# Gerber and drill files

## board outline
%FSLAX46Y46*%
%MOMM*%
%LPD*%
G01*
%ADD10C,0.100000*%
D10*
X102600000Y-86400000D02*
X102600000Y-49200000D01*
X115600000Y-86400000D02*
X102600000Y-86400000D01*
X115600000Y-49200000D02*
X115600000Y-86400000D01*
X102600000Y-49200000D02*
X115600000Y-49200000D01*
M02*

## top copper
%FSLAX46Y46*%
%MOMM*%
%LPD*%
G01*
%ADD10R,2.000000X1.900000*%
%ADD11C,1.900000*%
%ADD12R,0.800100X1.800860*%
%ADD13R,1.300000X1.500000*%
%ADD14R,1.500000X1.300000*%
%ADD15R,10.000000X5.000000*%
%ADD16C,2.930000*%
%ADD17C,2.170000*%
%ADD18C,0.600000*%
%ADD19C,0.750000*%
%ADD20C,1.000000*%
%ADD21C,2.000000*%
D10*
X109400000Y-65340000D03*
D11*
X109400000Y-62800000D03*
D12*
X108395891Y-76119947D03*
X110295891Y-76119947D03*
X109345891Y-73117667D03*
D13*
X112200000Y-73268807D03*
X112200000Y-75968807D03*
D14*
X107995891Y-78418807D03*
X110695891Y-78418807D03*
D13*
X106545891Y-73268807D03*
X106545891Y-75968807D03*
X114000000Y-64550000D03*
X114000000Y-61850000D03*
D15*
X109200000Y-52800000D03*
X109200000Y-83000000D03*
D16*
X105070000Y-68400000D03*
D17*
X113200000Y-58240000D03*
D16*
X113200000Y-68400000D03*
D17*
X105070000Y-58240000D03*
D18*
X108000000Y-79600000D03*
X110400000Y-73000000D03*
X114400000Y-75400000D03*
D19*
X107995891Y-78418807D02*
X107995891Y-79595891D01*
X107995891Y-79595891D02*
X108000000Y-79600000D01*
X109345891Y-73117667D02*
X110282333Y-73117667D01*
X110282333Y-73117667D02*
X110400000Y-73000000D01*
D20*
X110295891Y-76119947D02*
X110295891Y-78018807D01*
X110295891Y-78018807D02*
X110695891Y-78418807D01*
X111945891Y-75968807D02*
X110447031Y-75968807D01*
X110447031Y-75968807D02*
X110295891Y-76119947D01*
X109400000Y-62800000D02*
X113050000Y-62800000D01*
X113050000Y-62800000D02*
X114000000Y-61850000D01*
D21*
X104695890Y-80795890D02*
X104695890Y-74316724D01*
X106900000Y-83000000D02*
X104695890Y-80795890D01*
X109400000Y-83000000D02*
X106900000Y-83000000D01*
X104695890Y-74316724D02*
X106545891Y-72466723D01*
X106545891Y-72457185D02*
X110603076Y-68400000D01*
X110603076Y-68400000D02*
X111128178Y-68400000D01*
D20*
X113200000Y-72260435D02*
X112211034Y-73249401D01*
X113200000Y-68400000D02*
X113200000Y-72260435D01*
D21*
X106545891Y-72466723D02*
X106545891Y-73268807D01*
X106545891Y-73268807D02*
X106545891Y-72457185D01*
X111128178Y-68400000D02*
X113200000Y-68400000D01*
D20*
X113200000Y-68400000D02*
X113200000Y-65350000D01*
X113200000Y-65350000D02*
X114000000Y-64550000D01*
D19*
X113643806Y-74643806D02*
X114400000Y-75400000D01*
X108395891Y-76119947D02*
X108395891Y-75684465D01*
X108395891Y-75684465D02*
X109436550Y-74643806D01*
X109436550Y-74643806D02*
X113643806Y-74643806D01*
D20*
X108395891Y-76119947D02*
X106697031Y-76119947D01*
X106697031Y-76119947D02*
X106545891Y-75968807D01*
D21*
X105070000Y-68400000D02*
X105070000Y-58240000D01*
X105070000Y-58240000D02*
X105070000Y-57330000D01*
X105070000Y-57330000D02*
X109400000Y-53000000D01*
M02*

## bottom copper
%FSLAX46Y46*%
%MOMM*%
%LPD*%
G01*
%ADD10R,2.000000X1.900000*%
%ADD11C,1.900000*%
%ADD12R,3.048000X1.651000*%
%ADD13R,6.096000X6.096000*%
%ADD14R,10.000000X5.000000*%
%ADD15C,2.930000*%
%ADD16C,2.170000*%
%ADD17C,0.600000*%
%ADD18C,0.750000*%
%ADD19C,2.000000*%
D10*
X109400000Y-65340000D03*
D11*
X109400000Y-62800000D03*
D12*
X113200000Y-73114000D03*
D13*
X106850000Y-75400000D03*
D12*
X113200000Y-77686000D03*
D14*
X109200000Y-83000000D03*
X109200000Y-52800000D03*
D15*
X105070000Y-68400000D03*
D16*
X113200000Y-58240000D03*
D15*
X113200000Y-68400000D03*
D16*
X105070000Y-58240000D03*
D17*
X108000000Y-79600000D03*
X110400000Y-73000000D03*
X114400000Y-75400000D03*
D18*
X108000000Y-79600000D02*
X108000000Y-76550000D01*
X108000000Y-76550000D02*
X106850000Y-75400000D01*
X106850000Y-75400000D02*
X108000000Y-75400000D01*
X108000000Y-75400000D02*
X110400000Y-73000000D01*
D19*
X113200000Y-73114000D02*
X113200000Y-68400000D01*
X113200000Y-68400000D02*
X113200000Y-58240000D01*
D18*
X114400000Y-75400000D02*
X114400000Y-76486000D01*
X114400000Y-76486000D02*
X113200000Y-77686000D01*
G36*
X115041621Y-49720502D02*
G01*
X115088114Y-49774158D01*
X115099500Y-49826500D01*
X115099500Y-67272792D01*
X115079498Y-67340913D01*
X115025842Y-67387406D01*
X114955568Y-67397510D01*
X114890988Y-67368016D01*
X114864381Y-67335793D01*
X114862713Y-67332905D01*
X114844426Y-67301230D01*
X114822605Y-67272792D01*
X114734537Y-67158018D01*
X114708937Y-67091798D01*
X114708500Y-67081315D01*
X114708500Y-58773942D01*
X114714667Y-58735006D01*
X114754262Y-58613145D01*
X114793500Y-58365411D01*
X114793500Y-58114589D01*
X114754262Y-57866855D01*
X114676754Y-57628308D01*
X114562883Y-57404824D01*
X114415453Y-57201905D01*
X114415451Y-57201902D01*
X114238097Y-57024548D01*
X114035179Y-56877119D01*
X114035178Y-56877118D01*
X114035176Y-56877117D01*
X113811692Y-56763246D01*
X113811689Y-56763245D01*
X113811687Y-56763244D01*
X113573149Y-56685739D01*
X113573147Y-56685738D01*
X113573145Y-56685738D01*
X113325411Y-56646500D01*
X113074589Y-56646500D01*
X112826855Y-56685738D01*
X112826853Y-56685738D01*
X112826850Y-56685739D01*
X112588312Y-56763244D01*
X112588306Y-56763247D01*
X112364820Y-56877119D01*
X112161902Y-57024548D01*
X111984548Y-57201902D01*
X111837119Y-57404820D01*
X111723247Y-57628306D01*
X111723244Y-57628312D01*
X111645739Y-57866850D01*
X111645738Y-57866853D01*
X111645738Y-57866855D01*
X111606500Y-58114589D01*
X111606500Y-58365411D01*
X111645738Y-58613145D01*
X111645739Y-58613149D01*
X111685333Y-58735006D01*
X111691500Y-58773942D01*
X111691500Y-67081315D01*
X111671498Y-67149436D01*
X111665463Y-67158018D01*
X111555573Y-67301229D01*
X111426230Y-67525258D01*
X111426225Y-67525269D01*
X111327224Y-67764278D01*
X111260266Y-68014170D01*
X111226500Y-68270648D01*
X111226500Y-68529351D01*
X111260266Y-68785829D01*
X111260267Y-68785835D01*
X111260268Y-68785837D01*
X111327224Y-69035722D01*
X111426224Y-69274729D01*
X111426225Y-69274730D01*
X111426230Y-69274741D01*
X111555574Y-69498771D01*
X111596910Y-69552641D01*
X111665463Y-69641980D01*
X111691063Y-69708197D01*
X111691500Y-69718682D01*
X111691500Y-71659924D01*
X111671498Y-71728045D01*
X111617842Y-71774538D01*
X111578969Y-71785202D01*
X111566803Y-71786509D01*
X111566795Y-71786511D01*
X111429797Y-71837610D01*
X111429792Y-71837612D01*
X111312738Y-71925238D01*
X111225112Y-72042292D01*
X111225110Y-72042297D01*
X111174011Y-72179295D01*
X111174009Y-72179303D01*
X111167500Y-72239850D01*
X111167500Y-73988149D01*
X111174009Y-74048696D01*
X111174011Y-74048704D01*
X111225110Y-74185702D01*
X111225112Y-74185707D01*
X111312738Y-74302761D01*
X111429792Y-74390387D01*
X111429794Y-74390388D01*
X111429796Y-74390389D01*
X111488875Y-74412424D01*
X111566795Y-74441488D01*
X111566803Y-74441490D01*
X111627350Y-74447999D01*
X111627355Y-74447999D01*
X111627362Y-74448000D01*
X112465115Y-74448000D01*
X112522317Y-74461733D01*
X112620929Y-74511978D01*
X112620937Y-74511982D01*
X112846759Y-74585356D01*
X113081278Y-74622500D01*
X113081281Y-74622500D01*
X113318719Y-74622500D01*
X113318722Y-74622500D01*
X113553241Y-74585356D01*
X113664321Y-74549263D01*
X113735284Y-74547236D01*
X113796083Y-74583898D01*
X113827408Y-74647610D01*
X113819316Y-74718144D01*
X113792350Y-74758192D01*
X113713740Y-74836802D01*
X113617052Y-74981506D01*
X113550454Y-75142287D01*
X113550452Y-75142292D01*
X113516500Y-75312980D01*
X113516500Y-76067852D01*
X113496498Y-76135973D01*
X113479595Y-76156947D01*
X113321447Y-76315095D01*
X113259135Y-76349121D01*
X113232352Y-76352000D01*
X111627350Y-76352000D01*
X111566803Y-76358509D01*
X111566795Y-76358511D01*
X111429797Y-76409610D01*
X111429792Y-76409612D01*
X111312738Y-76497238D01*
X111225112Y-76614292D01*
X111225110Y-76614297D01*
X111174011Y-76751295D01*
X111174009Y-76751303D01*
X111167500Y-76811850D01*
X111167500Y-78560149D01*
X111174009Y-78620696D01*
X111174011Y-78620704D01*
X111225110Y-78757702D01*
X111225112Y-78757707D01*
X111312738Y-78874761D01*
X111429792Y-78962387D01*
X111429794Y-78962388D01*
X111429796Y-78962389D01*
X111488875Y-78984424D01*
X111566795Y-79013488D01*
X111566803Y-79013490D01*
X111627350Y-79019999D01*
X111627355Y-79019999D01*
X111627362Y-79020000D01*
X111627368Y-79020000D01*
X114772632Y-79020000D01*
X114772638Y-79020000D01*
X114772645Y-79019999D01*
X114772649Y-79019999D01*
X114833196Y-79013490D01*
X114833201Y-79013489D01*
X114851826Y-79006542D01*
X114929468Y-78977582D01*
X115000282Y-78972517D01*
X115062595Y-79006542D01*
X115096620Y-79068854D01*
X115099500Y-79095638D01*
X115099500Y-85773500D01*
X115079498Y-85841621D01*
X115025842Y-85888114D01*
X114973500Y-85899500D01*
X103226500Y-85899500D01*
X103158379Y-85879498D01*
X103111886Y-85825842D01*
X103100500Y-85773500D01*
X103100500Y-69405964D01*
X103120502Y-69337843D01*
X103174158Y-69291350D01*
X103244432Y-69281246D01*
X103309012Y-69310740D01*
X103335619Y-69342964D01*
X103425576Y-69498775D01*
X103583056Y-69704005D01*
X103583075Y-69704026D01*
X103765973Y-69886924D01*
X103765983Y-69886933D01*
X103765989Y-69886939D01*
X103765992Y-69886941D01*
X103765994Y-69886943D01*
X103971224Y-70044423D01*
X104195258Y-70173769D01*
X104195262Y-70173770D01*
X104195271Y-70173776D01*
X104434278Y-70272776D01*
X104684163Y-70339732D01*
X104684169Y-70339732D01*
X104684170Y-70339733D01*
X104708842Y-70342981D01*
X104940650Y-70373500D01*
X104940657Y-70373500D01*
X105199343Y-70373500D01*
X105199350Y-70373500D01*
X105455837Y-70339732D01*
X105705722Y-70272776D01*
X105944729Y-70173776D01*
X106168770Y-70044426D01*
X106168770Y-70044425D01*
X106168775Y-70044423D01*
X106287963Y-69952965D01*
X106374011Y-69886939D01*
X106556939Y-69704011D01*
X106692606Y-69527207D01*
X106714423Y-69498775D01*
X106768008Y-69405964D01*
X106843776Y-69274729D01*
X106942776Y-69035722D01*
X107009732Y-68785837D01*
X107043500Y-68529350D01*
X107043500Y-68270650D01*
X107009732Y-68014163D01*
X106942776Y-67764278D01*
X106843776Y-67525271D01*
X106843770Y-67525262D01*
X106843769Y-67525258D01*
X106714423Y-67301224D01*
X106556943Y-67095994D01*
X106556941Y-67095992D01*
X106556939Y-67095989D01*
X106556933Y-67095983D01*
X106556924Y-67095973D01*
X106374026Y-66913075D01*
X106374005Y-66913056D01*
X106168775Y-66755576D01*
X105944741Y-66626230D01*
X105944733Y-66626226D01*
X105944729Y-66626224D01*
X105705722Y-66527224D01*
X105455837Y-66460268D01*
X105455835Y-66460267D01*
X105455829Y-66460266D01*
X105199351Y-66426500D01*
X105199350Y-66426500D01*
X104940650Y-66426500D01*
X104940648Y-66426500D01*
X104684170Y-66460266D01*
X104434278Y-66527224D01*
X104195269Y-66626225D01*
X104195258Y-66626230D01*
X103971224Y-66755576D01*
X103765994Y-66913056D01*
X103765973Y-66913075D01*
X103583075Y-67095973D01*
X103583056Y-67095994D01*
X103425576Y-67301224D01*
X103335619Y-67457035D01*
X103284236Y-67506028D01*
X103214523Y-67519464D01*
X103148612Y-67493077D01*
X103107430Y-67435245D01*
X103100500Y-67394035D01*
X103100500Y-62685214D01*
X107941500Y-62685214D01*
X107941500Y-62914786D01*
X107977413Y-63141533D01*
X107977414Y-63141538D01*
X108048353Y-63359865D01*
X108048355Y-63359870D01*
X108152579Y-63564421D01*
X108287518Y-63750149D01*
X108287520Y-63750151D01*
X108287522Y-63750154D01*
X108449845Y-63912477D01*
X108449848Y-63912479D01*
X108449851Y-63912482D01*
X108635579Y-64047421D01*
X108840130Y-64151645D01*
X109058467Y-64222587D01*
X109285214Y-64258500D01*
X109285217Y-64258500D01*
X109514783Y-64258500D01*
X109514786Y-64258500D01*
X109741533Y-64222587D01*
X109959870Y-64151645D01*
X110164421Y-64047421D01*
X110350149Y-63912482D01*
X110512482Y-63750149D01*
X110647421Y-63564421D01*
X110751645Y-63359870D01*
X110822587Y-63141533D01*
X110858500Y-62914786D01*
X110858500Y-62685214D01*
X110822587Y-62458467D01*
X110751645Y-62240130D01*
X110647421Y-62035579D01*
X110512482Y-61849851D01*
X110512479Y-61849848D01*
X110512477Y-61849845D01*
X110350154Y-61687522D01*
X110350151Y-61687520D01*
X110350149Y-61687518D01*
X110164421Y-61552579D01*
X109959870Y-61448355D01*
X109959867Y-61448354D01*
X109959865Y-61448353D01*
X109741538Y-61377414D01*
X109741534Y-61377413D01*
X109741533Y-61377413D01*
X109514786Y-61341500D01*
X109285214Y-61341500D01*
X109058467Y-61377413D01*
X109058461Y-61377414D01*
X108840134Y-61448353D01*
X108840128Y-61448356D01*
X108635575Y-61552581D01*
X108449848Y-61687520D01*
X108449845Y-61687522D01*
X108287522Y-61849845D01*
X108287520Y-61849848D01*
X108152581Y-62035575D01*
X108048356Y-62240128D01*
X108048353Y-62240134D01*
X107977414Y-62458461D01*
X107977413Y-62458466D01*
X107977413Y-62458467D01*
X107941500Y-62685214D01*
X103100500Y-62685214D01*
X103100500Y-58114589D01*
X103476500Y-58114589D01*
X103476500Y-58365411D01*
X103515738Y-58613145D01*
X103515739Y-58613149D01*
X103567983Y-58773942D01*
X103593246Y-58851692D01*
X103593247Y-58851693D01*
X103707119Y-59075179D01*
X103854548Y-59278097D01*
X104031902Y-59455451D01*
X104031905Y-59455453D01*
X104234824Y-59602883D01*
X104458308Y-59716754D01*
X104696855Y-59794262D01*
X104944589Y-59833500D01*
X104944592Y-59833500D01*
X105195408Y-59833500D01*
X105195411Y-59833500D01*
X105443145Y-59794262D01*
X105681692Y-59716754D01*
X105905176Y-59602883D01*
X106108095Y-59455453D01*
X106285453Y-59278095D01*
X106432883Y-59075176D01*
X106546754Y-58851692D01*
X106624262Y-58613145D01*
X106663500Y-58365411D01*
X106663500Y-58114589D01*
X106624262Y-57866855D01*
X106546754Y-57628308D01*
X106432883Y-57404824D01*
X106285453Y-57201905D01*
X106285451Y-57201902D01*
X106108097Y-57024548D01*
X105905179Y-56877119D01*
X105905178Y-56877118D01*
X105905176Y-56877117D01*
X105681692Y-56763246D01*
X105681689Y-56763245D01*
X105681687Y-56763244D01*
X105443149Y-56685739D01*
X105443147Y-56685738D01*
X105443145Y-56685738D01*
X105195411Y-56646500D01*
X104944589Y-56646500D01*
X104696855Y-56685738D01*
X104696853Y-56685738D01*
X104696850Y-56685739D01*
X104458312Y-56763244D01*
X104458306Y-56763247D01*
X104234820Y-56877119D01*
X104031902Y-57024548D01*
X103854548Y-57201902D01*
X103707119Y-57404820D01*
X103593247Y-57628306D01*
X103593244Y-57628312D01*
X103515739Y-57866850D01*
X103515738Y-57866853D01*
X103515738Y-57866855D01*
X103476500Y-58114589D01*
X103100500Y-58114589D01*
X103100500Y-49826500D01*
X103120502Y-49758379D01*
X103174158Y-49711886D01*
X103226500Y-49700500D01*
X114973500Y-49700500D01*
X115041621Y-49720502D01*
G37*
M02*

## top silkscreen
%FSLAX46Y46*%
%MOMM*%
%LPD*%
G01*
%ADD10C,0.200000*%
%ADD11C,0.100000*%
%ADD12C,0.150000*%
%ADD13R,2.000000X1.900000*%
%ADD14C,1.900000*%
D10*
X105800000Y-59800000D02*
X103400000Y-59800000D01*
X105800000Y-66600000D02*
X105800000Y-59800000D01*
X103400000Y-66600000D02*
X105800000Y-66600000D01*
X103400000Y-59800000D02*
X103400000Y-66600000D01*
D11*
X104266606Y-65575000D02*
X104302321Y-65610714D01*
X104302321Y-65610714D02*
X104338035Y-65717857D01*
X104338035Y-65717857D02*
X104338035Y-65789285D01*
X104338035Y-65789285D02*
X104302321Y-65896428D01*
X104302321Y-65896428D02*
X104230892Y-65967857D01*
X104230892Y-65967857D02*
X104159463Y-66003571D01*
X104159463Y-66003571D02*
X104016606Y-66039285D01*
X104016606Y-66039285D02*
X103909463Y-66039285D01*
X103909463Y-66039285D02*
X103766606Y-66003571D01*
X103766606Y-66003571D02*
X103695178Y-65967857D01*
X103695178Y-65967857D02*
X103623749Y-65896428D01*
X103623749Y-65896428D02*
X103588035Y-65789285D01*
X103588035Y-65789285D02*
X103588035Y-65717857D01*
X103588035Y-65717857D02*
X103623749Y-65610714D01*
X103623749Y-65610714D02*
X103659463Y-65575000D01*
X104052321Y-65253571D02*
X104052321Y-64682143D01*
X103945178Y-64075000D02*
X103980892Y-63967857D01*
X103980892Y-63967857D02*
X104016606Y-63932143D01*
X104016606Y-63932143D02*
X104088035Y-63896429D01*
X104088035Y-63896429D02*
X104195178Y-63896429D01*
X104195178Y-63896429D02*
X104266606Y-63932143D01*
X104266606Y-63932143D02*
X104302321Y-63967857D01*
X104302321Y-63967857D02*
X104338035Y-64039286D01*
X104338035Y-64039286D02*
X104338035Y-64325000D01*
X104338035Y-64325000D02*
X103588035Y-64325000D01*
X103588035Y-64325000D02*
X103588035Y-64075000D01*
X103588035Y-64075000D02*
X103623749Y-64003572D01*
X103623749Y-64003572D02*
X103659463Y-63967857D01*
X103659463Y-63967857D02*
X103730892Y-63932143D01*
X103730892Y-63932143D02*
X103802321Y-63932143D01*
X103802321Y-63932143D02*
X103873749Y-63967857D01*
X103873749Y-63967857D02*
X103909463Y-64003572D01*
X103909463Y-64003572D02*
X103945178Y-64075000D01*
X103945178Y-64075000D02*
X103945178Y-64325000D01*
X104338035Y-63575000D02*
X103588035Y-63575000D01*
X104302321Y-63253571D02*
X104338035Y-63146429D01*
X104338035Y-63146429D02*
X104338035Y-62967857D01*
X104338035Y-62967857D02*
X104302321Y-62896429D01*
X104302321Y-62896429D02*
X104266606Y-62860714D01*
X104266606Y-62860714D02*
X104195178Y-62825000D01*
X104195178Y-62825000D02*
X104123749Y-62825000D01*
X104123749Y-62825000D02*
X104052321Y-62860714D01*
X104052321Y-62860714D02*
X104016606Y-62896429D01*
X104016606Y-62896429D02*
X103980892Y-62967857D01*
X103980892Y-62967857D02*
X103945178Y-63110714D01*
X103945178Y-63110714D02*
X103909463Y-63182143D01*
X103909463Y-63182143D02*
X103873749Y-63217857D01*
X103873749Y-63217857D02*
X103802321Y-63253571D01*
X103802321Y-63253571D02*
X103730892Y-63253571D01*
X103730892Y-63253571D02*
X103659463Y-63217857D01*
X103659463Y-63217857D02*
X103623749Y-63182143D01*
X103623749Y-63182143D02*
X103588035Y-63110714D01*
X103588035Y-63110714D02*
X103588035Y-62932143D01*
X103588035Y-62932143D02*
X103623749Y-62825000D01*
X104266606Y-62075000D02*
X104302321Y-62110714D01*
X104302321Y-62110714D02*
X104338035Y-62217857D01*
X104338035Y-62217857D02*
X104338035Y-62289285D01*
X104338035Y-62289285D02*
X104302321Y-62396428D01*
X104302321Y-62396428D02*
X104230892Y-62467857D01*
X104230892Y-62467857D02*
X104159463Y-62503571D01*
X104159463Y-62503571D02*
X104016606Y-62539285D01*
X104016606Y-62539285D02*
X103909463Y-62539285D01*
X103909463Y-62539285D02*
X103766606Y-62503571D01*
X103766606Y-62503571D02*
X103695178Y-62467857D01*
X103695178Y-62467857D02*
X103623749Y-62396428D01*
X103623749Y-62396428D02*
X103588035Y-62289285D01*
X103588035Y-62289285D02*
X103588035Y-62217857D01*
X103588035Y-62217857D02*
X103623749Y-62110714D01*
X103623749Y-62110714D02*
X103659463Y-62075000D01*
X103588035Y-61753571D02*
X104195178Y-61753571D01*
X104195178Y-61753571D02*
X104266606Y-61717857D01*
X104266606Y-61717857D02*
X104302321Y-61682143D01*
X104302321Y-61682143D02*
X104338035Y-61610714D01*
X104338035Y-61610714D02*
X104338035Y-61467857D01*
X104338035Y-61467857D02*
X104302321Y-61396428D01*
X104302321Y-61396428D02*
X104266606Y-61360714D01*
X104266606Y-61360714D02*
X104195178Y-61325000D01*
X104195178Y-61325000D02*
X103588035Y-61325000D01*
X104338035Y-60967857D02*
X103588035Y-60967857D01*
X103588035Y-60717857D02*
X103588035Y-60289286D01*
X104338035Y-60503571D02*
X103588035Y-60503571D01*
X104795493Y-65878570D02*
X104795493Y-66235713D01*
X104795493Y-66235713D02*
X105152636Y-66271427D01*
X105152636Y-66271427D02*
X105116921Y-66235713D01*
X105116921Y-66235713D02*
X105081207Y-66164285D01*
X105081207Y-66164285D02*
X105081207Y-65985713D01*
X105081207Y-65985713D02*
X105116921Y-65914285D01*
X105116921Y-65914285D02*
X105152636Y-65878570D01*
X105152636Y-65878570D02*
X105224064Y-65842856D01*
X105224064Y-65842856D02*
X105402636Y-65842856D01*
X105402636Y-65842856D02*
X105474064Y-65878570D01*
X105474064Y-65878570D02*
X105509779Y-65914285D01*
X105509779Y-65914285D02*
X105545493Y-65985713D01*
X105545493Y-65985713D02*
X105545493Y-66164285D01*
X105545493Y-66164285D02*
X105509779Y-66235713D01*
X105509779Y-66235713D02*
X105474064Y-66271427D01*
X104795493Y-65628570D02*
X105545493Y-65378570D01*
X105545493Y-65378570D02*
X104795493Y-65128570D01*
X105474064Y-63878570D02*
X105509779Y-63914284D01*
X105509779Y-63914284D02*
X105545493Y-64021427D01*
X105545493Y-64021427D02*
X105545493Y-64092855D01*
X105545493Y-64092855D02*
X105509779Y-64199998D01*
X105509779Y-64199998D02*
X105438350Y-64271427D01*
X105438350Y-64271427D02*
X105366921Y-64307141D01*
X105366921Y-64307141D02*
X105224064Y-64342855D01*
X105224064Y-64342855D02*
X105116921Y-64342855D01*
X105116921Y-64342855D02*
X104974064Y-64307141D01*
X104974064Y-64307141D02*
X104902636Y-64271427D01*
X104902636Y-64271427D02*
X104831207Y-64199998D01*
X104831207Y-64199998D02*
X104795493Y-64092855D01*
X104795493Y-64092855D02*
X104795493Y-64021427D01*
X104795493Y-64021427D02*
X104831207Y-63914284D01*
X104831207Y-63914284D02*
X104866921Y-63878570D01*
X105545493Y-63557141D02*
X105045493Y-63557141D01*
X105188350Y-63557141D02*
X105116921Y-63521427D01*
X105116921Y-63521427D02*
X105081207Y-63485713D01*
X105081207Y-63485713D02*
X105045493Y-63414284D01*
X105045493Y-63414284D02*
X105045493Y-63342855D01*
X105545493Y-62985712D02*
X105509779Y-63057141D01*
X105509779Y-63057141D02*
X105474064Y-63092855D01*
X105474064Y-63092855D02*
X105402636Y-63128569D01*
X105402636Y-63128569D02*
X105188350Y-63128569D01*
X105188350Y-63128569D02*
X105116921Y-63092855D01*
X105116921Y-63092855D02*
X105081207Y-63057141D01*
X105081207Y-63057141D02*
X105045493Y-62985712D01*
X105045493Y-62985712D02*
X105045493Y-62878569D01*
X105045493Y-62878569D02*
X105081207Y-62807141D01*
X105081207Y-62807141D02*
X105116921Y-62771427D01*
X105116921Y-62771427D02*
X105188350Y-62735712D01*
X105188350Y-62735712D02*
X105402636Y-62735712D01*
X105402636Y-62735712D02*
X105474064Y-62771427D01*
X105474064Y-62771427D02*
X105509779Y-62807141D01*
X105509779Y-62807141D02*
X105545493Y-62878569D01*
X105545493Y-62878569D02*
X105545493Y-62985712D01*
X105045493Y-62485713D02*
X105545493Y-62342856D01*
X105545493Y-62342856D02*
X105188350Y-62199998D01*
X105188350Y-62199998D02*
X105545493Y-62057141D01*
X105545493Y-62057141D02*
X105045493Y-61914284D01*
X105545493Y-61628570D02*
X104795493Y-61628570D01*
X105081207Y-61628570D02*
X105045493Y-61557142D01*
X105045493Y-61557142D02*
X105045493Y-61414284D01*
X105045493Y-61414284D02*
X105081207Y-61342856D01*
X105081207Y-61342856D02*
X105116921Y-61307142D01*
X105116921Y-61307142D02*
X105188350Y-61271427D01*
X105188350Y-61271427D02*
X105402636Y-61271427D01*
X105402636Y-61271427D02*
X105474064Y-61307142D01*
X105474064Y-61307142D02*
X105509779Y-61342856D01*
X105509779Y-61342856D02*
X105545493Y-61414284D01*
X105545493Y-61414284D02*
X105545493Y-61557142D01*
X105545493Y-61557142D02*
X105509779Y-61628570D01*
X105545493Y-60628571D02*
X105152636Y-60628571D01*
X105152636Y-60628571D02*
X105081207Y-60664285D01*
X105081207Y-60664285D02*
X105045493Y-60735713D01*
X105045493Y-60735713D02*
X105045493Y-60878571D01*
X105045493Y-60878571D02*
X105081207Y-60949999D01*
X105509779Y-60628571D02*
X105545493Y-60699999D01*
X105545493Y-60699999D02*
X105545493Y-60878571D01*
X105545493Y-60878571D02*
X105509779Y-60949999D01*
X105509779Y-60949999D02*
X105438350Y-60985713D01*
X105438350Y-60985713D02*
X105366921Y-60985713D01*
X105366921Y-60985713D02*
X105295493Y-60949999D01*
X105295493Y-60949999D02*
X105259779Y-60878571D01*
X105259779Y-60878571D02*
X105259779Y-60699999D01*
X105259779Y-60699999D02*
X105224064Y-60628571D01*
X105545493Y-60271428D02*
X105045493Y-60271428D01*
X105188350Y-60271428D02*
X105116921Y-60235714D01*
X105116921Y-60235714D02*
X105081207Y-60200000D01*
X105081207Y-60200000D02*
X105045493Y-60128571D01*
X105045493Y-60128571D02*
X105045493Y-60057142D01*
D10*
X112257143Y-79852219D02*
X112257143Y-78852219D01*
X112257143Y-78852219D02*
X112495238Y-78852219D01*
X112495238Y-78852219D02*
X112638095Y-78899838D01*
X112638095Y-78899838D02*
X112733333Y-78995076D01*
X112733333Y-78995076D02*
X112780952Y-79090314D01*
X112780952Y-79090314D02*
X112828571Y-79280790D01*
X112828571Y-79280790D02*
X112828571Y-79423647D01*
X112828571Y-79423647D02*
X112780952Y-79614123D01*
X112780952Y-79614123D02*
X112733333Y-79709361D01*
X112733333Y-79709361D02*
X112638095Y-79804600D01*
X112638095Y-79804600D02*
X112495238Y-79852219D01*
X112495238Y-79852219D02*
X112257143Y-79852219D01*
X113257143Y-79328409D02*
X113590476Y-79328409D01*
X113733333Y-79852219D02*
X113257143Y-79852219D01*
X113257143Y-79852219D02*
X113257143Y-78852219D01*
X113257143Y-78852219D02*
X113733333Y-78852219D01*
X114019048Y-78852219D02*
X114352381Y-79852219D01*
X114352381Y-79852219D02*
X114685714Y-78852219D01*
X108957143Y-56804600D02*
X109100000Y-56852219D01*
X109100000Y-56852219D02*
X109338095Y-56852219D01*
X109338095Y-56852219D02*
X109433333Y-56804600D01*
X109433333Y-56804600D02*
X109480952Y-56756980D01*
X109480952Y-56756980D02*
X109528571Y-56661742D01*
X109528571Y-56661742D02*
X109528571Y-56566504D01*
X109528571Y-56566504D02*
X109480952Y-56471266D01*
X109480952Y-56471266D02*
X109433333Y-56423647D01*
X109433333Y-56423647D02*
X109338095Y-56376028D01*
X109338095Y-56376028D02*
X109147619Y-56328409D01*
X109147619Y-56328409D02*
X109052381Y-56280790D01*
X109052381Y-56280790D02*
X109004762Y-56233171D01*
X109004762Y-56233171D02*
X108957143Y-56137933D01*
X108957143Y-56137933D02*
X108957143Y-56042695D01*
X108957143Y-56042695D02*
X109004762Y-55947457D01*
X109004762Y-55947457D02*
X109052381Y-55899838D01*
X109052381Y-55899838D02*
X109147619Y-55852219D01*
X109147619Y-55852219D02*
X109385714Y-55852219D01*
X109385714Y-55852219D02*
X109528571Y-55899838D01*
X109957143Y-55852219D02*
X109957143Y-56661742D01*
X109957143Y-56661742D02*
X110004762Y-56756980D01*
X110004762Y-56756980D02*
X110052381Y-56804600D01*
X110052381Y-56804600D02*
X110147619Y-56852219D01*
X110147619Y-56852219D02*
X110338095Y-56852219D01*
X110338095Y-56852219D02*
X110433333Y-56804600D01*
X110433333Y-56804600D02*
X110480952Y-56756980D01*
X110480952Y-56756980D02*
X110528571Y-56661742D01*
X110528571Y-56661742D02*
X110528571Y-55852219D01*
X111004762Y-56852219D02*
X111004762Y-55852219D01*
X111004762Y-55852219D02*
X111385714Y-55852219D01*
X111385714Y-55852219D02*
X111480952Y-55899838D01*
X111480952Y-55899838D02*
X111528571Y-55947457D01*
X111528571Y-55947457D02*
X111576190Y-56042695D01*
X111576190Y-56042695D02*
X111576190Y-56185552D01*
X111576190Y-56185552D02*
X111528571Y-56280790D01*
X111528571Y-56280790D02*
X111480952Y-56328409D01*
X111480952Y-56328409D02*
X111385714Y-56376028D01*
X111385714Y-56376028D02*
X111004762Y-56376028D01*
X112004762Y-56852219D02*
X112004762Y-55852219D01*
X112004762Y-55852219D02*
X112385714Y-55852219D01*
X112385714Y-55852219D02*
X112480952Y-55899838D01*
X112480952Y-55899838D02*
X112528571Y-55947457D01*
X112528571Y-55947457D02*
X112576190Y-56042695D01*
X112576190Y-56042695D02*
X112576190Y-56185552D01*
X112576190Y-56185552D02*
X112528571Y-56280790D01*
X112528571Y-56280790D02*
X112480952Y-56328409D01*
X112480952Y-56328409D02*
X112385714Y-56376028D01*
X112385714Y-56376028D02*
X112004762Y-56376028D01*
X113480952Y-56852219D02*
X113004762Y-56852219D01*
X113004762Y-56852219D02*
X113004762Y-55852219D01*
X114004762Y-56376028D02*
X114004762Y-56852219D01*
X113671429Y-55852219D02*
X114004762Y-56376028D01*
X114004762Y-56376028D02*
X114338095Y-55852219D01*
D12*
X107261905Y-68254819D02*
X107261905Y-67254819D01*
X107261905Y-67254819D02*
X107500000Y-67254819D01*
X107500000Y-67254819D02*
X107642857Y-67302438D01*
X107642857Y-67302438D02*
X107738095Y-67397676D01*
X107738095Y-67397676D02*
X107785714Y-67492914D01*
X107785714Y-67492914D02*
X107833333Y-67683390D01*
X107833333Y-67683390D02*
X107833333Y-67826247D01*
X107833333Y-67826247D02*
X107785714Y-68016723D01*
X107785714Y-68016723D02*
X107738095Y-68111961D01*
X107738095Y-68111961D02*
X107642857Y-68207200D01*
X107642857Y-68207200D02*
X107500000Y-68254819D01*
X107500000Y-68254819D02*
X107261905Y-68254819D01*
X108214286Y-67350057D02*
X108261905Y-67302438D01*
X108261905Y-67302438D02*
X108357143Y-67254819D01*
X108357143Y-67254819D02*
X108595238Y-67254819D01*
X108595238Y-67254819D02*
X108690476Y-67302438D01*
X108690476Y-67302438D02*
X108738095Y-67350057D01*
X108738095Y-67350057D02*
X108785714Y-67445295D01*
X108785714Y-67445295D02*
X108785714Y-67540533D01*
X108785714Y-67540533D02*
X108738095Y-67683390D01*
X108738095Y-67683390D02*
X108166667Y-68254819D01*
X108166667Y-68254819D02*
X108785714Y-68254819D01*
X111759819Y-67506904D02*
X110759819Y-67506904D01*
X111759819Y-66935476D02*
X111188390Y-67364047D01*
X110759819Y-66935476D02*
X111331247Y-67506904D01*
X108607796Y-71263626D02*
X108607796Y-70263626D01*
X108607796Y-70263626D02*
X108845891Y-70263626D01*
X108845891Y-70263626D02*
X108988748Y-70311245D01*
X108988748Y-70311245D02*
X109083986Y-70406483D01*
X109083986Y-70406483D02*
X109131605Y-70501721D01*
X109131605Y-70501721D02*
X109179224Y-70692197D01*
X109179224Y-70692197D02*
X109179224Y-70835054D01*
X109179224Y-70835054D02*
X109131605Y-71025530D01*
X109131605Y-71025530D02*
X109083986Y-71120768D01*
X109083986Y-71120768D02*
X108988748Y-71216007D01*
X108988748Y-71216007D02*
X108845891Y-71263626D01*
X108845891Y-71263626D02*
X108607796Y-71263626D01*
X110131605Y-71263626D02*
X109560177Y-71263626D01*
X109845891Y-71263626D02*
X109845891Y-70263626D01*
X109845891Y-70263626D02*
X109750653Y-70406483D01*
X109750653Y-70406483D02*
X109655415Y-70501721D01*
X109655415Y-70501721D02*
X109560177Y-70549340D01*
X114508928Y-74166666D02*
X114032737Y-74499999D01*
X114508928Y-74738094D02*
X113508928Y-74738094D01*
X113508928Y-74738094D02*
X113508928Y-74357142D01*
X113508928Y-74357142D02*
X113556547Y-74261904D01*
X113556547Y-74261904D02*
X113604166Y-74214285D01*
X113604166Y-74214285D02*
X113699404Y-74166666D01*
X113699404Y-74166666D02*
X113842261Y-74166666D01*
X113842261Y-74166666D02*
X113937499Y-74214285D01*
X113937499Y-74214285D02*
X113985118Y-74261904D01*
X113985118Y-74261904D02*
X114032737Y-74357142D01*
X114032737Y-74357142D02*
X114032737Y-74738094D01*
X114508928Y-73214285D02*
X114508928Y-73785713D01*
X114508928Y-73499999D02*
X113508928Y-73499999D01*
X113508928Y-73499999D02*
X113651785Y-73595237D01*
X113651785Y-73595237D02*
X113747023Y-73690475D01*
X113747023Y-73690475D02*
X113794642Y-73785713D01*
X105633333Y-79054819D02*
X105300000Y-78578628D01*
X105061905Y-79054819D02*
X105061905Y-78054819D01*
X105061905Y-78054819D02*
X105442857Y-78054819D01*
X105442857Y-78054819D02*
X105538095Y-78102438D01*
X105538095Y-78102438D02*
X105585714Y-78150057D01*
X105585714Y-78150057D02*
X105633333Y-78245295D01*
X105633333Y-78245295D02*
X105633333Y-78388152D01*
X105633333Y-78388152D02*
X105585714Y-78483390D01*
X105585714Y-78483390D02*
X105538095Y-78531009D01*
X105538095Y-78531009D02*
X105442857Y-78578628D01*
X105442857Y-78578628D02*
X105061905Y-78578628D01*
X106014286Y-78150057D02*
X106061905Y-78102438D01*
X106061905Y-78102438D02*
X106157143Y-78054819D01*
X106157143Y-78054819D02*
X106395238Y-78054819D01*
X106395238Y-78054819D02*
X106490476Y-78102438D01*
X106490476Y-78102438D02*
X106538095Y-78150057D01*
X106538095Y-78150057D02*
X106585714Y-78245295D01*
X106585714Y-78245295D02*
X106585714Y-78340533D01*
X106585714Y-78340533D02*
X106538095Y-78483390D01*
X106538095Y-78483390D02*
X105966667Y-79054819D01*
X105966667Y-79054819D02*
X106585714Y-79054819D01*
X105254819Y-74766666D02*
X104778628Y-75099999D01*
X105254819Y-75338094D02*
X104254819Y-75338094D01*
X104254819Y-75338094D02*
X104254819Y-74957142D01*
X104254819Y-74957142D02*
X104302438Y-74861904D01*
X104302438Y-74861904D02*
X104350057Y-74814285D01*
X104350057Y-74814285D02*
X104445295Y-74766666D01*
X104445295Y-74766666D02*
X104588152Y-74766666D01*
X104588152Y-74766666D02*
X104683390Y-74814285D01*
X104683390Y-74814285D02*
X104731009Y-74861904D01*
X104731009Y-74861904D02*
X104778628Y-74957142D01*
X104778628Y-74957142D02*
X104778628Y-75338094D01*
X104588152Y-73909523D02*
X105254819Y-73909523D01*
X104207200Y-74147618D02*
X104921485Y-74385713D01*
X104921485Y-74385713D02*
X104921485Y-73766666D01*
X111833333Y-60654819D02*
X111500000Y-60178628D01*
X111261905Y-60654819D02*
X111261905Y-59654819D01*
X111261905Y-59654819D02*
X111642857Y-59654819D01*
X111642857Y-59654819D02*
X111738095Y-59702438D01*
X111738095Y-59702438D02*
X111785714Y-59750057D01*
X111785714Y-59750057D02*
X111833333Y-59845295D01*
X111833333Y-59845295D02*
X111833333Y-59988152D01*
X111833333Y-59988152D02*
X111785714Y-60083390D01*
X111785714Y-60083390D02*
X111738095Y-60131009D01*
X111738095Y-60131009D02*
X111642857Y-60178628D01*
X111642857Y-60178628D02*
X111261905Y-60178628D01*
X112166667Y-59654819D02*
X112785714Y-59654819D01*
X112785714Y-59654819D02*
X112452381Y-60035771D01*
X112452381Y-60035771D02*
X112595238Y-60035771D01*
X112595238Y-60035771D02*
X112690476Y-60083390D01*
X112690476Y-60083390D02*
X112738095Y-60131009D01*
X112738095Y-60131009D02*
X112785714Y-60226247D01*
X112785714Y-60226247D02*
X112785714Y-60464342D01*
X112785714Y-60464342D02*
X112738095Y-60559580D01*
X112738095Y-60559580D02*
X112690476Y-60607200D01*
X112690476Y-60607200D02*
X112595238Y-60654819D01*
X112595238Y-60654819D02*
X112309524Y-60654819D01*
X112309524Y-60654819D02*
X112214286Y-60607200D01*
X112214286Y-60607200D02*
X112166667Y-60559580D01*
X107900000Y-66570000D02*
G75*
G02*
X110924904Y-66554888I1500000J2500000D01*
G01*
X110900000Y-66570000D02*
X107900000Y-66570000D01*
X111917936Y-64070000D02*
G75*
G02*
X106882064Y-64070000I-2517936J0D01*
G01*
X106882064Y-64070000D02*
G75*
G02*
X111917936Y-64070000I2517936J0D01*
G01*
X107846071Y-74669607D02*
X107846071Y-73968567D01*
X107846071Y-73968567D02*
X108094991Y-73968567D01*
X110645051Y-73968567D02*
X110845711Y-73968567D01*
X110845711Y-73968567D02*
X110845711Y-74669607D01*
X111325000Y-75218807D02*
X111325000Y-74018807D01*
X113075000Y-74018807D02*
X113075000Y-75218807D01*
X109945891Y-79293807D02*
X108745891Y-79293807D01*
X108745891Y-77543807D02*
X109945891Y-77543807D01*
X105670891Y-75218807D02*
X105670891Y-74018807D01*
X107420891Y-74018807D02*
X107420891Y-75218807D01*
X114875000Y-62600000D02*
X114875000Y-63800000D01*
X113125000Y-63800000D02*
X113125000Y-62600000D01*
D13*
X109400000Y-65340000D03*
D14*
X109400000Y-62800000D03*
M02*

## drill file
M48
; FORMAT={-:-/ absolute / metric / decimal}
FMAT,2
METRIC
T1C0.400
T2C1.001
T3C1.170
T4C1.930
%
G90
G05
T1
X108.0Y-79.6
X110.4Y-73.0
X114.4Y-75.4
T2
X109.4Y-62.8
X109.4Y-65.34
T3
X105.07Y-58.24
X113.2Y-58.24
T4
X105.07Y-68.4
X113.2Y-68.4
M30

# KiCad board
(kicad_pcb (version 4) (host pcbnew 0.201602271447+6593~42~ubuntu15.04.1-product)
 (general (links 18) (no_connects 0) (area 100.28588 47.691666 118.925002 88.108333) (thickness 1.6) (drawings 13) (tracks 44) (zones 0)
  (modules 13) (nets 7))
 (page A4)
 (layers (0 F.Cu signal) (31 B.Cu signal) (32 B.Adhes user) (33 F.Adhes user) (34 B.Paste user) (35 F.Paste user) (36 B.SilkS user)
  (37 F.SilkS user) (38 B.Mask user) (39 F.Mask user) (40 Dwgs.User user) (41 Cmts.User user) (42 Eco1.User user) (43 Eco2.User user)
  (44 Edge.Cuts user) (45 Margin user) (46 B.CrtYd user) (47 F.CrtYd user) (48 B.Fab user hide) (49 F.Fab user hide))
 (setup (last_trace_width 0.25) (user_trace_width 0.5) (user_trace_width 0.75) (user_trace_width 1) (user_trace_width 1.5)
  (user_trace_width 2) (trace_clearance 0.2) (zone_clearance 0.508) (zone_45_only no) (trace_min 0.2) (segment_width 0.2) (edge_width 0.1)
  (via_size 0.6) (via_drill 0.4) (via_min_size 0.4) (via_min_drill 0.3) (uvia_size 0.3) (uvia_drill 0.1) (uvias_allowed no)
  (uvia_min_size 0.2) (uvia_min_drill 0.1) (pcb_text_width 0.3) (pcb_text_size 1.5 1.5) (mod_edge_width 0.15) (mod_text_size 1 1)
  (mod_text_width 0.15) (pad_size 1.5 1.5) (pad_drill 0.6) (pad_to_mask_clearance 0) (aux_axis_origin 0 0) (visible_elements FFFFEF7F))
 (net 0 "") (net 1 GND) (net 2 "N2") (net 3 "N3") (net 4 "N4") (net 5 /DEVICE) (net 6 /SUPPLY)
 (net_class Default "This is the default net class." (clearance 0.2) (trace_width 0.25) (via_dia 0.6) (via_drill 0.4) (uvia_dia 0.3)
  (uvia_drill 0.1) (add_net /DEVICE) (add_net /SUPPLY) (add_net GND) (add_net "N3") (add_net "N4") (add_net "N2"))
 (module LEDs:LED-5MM (layer F.Cu) (at 109.4 65.34 90)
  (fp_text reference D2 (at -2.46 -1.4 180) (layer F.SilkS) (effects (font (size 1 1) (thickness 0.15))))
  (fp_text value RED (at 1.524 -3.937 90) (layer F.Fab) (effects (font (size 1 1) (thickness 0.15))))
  (fp_arc (start 1.27 0) (end -1.23 -1.5) (angle 297.5) (layer F.SilkS) (width 0.15))
  (fp_line (start -1.23 1.5) (end -1.23 -1.5) (layer F.SilkS) (width 0.15))
  (fp_circle (center 1.27 0) (end 0.97 -2.5) (layer F.SilkS) (width 0.15))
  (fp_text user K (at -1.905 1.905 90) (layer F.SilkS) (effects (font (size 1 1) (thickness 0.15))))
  (pad 1 thru_hole rect (at 0 0 180) (size 2 1.9) (drill 1.00076) (layers *.Cu *.Mask F.SilkS) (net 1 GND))
  (pad 2 thru_hole circle (at 2.54 0 90) (size 1.9 1.9) (drill 1.00076) (layers *.Cu *.Mask F.SilkS) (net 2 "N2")))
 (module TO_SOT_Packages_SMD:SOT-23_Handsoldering (layer F.Cu) (at 109.345891 74.618807)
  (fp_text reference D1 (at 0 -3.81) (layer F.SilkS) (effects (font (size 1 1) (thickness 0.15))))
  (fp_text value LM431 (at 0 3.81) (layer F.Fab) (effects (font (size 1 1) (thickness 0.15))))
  (fp_line (start -1.49982 0.0508) (end -1.49982 -0.65024) (layer F.SilkS) (width 0.15))
  (fp_line (start -1.49982 -0.65024) (end -1.2509 -0.65024) (layer F.SilkS) (width 0.15))
  (fp_line (start 1.29916 -0.65024) (end 1.49982 -0.65024) (layer F.SilkS) (width 0.15))
  (fp_line (start 1.49982 -0.65024) (end 1.49982 0.0508) (layer F.SilkS) (width 0.15))
  (pad 1 smd rect (at -0.95 1.50114) (size 0.8001 1.80086) (layers F.Cu F.Paste F.Mask) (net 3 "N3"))
  (pad 2 smd rect (at 0.95 1.50114) (size 0.8001 1.80086) (layers F.Cu F.Paste F.Mask) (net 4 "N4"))
  (pad 3 smd rect (at 0 -1.50114) (size 0.8001 1.80086) (layers F.Cu F.Paste F.Mask) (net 1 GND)))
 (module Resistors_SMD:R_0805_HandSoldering (layer F.Cu) (at 112.2 74.618807 270)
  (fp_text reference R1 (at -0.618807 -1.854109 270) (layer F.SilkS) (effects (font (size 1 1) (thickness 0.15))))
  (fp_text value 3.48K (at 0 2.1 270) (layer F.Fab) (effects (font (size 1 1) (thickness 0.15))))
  (fp_line (start 0.6 0.875) (end -0.6 0.875) (layer F.SilkS) (width 0.15))
  (fp_line (start -0.6 -0.875) (end 0.6 -0.875) (layer F.SilkS) (width 0.15))
  (pad 1 smd rect (at -1.35 0 270) (size 1.5 1.3) (layers F.Cu F.Paste F.Mask) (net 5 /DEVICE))
  (pad 2 smd rect (at 1.35 0 270) (size 1.5 1.3) (layers F.Cu F.Paste F.Mask) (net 4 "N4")))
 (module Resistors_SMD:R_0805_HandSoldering (layer F.Cu) (at 109.345891 78.418807)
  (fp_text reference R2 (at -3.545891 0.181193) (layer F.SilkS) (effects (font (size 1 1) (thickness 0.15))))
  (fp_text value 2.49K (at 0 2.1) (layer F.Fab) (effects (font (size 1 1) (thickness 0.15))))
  (fp_line (start 0.6 0.875) (end -0.6 0.875) (layer F.SilkS) (width 0.15))
  (fp_line (start -0.6 -0.875) (end 0.6 -0.875) (layer F.SilkS) (width 0.15))
  (pad 1 smd rect (at -1.35 0) (size 1.5 1.3) (layers F.Cu F.Paste F.Mask) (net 1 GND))
  (pad 2 smd rect (at 1.35 0) (size 1.5 1.3) (layers F.Cu F.Paste F.Mask) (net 4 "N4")))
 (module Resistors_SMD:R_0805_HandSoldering (layer F.Cu) (at 106.545891 74.618807 270)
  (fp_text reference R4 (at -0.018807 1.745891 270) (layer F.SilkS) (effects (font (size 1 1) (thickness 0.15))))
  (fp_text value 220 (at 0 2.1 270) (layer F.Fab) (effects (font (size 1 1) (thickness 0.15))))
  (fp_line (start 0.6 0.875) (end -0.6 0.875) (layer F.SilkS) (width 0.15))
  (fp_line (start -0.6 -0.875) (end 0.6 -0.875) (layer F.SilkS) (width 0.15))
  (pad 1 smd rect (at -1.35 0 270) (size 1.5 1.3) (layers F.Cu F.Paste F.Mask) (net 5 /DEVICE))
  (pad 2 smd rect (at 1.35 0 270) (size 1.5 1.3) (layers F.Cu F.Paste F.Mask) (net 3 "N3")))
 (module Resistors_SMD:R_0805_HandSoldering (layer F.Cu) (at 114 63.2 90)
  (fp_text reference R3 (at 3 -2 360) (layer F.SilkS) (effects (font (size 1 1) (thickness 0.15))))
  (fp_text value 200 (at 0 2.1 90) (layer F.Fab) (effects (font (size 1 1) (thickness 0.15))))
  (fp_line (start 0.6 0.875) (end -0.6 0.875) (layer F.SilkS) (width 0.15))
  (fp_line (start -0.6 -0.875) (end 0.6 -0.875) (layer F.SilkS) (width 0.15))
  (pad 1 smd rect (at -1.35 0 90) (size 1.5 1.3) (layers F.Cu F.Paste F.Mask) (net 5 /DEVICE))
  (pad 2 smd rect (at 1.35 0 90) (size 1.5 1.3) (layers F.Cu F.Paste F.Mask) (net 2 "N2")))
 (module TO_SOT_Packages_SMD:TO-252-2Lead (layer B.Cu) (at 113.2 75.4 270)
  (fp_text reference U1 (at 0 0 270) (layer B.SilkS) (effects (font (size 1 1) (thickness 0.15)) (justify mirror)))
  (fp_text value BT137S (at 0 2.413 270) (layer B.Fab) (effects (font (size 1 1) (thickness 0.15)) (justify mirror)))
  (pad 1 smd rect (at -2.286 0 270) (size 1.651 3.048) (layers B.Cu B.Paste B.Mask) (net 5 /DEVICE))
  (pad 2 smd rect (at 0 6.35 270) (size 6.096 6.096) (layers B.Cu B.Paste B.Mask) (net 1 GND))
  (pad 3 smd rect (at 2.286 0 270) (size 1.651 3.048) (layers B.Cu B.Paste B.Mask) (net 3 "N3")))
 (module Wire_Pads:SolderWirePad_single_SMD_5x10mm (layer F.Cu) (at 109.2 52.8 90)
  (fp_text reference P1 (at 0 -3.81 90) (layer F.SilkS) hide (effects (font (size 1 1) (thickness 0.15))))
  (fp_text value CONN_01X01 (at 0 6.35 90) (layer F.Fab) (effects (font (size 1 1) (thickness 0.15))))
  (pad 1 smd rect (at 0 0 90) (size 5 10) (layers F.Cu F.Paste F.Mask) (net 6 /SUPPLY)))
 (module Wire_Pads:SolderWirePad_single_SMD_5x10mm (layer F.Cu) (at 109.2 83 90)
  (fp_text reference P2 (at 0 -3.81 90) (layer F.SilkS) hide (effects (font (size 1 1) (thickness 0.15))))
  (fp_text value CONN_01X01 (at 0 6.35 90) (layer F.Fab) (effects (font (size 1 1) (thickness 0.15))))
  (pad 1 smd rect (at 0 0 90) (size 5 10) (layers F.Cu F.Paste F.Mask) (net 5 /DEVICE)))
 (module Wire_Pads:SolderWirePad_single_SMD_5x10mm (layer B.Cu) (at 109.2 83 90)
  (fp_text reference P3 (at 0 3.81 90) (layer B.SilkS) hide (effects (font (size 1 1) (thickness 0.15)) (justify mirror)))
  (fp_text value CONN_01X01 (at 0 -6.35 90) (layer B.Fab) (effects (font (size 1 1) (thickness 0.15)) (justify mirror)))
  (pad 1 smd rect (at 0 0 90) (size 5 10) (layers B.Cu B.Paste B.Mask) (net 1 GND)))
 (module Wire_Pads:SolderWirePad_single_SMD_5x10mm (layer B.Cu) (at 109.2 52.8 90)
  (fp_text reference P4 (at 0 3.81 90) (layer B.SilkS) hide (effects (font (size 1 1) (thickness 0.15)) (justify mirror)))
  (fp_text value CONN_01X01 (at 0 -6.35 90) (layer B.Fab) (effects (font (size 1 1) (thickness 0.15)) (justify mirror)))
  (pad 1 smd rect (at 0 0 90) (size 5 10) (layers B.Cu B.Paste B.Mask) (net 1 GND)))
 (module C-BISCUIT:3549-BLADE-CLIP (layer B.Cu) (at 109.135 63.32)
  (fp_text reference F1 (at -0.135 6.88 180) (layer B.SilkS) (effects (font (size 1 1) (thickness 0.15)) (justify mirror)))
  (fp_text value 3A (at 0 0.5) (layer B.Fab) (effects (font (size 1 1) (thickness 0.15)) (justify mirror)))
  (pad 1 thru_hole circle (at -4.065 5.08) (size 2.93 2.93) (drill 1.93) (layers *.Cu *.Mask B.SilkS) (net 6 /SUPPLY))
  (pad 2 thru_hole circle (at 4.065 -5.08) (size 2.17 2.17) (drill 1.17) (layers *.Cu *.Mask B.SilkS) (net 5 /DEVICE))
  (pad 2 thru_hole circle (at 4.065 5.08) (size 2.93 2.93) (drill 1.93) (layers *.Cu *.Mask B.SilkS) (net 5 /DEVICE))
  (pad 1 thru_hole circle (at -4.065 -5.08) (size 2.17 2.17) (drill 1.17) (layers *.Cu *.Mask B.SilkS) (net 6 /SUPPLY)))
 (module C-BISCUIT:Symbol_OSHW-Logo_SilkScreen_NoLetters (layer B.Cu) (at 105.8 63.2 270)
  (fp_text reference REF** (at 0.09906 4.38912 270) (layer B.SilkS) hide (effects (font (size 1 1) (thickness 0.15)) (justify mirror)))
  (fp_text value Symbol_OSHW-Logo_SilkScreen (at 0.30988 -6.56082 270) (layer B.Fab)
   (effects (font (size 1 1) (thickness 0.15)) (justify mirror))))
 (gr_line (start 105.8 59.8) (end 103.4 59.8) (layer F.SilkS) (width 0.2))
 (gr_line (start 105.8 66.6) (end 105.8 59.8) (layer F.SilkS) (width 0.2))
 (gr_line (start 103.4 66.6) (end 105.8 66.6) (layer F.SilkS) (width 0.2))
 (gr_line (start 103.4 59.8) (end 103.4 66.6) (layer F.SilkS) (width 0.2))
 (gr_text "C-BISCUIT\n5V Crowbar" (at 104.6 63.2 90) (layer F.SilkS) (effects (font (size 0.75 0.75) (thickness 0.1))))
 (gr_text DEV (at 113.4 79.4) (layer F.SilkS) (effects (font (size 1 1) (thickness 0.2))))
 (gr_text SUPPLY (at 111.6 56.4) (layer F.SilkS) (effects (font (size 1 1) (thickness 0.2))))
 (gr_line (start 102.6 86.4) (end 102.6 49.2) (layer Edge.Cuts) (width 0.1))
 (gr_line (start 115.6 86.4) (end 102.6 86.4) (layer Edge.Cuts) (width 0.1))
 (gr_line (start 115.6 49.2) (end 115.6 86.4) (layer Edge.Cuts) (width 0.1))
 (gr_line (start 102.6 49.2) (end 115.6 49.2) (layer Edge.Cuts) (width 0.1))
 (segment (start 100.8 48.8) (end 118.6 48.8) (width 0.25) (layer Dwgs.User) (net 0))
 (segment (start 108 79.6) (end 108 76.55) (width 0.75) (layer B.Cu) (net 1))
 (segment (start 108 76.55) (end 106.85 75.4) (width 0.75) (layer B.Cu) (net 1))
 (segment (start 107.995891 78.418807) (end 107.995891 79.595891) (width 0.75) (layer F.Cu) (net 1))
 (segment (start 107.995891 79.595891) (end 108 79.6) (width 0.75) (layer F.Cu) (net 1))
 (via (at 108 79.6) (size 0.6) (drill 0.4) (layers F.Cu B.Cu) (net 1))
 (segment (start 106.85 75.4) (end 108 75.4) (width 0.75) (layer B.Cu) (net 1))
 (segment (start 108 75.4) (end 110.4 73) (width 0.75) (layer B.Cu) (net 1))
 (segment (start 109.345891 73.117667) (end 110.282333 73.117667) (width 0.75) (layer F.Cu) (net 1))
 (via (at 110.4 73) (size 0.6) (drill 0.4) (layers F.Cu B.Cu) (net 1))
 (segment (start 110.282333 73.117667) (end 110.4 73) (width 0.75) (layer F.Cu) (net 1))
 (segment (start 110.295891 76.119947) (end 110.295891 78.018807) (width 1) (layer F.Cu) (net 4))
 (segment (start 110.295891 78.018807) (end 110.695891 78.418807) (width 1) (layer F.Cu) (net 4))
 (segment (start 111.945891 75.968807) (end 110.447031 75.968807) (width 1) (layer F.Cu) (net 4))
 (segment (start 110.447031 75.968807) (end 110.295891 76.119947) (width 1) (layer F.Cu) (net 4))
 (segment (start 109.4 62.8) (end 113.05 62.8) (width 1) (layer F.Cu) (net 2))
 (segment (start 113.05 62.8) (end 114 61.85) (width 1) (layer F.Cu) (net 2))
 (segment (start 104.69589 80.79589) (end 104.69589 74.316724) (width 2) (layer F.Cu) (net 5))
 (segment (start 106.9 83) (end 104.69589 80.79589) (width 2) (layer F.Cu) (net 5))
 (segment (start 109.4 83) (end 106.9 83) (width 2) (layer F.Cu) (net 5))
 (segment (start 104.69589 74.316724) (end 106.545891 72.466723) (width 2) (layer F.Cu) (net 5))
 (segment (start 106.545891 72.457185) (end 110.603076 68.4) (width 2) (layer F.Cu) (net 5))
 (segment (start 110.603076 68.4) (end 111.128178 68.4) (width 2) (layer F.Cu) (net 5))
 (segment (start 113.2 72.260435) (end 112.211034 73.249401) (width 1) (layer F.Cu) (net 5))
 (segment (start 113.2 68.4) (end 113.2 72.260435) (width 1) (layer F.Cu) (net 5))
 (segment (start 106.545891 72.466723) (end 106.545891 73.268807) (width 2) (layer F.Cu) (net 5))
 (segment (start 106.545891 73.268807) (end 106.545891 72.457185) (width 2) (layer F.Cu) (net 5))
 (segment (start 111.128178 68.4) (end 113.2 68.4) (width 2) (layer F.Cu) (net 5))
 (segment (start 113.2 73.114) (end 113.2 68.4) (width 2) (layer B.Cu) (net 5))
 (segment (start 113.2 68.4) (end 113.2 65.35) (width 1) (layer F.Cu) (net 5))
 (segment (start 113.2 65.35) (end 114 64.55) (width 1) (layer F.Cu) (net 5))
 (segment (start 113.2 68.4) (end 113.2 58.24) (width 2) (layer B.Cu) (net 5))
 (segment (start 113.643806 74.643806) (end 114.4 75.4) (width 0.75) (layer F.Cu) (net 3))
 (segment (start 108.395891 76.119947) (end 108.395891 75.684465) (width 0.75) (layer F.Cu) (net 3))
 (segment (start 108.395891 75.684465) (end 109.43655 74.643806) (width 0.75) (layer F.Cu) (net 3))
 (segment (start 109.43655 74.643806) (end 113.643806 74.643806) (width 0.75) (layer F.Cu) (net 3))
 (segment (start 108.395891 76.119947) (end 106.697031 76.119947) (width 1) (layer F.Cu) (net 3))
 (segment (start 106.697031 76.119947) (end 106.545891 75.968807) (width 1) (layer F.Cu) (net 3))
 (segment (start 114.4 75.4) (end 114.4 76.486) (width 0.75) (layer B.Cu) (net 3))
 (via (at 114.4 75.4) (size 0.6) (drill 0.4) (layers F.Cu B.Cu) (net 3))
 (segment (start 114.4 76.486) (end 113.2 77.686) (width 0.75) (layer B.Cu) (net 3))
 (segment (start 105.07 68.4) (end 105.07 58.24) (width 2) (layer F.Cu) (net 6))
 (segment (start 105.07 58.24) (end 105.07 57.33) (width 2) (layer F.Cu) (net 6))
 (segment (start 105.07 57.33) (end 109.4 53) (width 2) (layer F.Cu) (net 6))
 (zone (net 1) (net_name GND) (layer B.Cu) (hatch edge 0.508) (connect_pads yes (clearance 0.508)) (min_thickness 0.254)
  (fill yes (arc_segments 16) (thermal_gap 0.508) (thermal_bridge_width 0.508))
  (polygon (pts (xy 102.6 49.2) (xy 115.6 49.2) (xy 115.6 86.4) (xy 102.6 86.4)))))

